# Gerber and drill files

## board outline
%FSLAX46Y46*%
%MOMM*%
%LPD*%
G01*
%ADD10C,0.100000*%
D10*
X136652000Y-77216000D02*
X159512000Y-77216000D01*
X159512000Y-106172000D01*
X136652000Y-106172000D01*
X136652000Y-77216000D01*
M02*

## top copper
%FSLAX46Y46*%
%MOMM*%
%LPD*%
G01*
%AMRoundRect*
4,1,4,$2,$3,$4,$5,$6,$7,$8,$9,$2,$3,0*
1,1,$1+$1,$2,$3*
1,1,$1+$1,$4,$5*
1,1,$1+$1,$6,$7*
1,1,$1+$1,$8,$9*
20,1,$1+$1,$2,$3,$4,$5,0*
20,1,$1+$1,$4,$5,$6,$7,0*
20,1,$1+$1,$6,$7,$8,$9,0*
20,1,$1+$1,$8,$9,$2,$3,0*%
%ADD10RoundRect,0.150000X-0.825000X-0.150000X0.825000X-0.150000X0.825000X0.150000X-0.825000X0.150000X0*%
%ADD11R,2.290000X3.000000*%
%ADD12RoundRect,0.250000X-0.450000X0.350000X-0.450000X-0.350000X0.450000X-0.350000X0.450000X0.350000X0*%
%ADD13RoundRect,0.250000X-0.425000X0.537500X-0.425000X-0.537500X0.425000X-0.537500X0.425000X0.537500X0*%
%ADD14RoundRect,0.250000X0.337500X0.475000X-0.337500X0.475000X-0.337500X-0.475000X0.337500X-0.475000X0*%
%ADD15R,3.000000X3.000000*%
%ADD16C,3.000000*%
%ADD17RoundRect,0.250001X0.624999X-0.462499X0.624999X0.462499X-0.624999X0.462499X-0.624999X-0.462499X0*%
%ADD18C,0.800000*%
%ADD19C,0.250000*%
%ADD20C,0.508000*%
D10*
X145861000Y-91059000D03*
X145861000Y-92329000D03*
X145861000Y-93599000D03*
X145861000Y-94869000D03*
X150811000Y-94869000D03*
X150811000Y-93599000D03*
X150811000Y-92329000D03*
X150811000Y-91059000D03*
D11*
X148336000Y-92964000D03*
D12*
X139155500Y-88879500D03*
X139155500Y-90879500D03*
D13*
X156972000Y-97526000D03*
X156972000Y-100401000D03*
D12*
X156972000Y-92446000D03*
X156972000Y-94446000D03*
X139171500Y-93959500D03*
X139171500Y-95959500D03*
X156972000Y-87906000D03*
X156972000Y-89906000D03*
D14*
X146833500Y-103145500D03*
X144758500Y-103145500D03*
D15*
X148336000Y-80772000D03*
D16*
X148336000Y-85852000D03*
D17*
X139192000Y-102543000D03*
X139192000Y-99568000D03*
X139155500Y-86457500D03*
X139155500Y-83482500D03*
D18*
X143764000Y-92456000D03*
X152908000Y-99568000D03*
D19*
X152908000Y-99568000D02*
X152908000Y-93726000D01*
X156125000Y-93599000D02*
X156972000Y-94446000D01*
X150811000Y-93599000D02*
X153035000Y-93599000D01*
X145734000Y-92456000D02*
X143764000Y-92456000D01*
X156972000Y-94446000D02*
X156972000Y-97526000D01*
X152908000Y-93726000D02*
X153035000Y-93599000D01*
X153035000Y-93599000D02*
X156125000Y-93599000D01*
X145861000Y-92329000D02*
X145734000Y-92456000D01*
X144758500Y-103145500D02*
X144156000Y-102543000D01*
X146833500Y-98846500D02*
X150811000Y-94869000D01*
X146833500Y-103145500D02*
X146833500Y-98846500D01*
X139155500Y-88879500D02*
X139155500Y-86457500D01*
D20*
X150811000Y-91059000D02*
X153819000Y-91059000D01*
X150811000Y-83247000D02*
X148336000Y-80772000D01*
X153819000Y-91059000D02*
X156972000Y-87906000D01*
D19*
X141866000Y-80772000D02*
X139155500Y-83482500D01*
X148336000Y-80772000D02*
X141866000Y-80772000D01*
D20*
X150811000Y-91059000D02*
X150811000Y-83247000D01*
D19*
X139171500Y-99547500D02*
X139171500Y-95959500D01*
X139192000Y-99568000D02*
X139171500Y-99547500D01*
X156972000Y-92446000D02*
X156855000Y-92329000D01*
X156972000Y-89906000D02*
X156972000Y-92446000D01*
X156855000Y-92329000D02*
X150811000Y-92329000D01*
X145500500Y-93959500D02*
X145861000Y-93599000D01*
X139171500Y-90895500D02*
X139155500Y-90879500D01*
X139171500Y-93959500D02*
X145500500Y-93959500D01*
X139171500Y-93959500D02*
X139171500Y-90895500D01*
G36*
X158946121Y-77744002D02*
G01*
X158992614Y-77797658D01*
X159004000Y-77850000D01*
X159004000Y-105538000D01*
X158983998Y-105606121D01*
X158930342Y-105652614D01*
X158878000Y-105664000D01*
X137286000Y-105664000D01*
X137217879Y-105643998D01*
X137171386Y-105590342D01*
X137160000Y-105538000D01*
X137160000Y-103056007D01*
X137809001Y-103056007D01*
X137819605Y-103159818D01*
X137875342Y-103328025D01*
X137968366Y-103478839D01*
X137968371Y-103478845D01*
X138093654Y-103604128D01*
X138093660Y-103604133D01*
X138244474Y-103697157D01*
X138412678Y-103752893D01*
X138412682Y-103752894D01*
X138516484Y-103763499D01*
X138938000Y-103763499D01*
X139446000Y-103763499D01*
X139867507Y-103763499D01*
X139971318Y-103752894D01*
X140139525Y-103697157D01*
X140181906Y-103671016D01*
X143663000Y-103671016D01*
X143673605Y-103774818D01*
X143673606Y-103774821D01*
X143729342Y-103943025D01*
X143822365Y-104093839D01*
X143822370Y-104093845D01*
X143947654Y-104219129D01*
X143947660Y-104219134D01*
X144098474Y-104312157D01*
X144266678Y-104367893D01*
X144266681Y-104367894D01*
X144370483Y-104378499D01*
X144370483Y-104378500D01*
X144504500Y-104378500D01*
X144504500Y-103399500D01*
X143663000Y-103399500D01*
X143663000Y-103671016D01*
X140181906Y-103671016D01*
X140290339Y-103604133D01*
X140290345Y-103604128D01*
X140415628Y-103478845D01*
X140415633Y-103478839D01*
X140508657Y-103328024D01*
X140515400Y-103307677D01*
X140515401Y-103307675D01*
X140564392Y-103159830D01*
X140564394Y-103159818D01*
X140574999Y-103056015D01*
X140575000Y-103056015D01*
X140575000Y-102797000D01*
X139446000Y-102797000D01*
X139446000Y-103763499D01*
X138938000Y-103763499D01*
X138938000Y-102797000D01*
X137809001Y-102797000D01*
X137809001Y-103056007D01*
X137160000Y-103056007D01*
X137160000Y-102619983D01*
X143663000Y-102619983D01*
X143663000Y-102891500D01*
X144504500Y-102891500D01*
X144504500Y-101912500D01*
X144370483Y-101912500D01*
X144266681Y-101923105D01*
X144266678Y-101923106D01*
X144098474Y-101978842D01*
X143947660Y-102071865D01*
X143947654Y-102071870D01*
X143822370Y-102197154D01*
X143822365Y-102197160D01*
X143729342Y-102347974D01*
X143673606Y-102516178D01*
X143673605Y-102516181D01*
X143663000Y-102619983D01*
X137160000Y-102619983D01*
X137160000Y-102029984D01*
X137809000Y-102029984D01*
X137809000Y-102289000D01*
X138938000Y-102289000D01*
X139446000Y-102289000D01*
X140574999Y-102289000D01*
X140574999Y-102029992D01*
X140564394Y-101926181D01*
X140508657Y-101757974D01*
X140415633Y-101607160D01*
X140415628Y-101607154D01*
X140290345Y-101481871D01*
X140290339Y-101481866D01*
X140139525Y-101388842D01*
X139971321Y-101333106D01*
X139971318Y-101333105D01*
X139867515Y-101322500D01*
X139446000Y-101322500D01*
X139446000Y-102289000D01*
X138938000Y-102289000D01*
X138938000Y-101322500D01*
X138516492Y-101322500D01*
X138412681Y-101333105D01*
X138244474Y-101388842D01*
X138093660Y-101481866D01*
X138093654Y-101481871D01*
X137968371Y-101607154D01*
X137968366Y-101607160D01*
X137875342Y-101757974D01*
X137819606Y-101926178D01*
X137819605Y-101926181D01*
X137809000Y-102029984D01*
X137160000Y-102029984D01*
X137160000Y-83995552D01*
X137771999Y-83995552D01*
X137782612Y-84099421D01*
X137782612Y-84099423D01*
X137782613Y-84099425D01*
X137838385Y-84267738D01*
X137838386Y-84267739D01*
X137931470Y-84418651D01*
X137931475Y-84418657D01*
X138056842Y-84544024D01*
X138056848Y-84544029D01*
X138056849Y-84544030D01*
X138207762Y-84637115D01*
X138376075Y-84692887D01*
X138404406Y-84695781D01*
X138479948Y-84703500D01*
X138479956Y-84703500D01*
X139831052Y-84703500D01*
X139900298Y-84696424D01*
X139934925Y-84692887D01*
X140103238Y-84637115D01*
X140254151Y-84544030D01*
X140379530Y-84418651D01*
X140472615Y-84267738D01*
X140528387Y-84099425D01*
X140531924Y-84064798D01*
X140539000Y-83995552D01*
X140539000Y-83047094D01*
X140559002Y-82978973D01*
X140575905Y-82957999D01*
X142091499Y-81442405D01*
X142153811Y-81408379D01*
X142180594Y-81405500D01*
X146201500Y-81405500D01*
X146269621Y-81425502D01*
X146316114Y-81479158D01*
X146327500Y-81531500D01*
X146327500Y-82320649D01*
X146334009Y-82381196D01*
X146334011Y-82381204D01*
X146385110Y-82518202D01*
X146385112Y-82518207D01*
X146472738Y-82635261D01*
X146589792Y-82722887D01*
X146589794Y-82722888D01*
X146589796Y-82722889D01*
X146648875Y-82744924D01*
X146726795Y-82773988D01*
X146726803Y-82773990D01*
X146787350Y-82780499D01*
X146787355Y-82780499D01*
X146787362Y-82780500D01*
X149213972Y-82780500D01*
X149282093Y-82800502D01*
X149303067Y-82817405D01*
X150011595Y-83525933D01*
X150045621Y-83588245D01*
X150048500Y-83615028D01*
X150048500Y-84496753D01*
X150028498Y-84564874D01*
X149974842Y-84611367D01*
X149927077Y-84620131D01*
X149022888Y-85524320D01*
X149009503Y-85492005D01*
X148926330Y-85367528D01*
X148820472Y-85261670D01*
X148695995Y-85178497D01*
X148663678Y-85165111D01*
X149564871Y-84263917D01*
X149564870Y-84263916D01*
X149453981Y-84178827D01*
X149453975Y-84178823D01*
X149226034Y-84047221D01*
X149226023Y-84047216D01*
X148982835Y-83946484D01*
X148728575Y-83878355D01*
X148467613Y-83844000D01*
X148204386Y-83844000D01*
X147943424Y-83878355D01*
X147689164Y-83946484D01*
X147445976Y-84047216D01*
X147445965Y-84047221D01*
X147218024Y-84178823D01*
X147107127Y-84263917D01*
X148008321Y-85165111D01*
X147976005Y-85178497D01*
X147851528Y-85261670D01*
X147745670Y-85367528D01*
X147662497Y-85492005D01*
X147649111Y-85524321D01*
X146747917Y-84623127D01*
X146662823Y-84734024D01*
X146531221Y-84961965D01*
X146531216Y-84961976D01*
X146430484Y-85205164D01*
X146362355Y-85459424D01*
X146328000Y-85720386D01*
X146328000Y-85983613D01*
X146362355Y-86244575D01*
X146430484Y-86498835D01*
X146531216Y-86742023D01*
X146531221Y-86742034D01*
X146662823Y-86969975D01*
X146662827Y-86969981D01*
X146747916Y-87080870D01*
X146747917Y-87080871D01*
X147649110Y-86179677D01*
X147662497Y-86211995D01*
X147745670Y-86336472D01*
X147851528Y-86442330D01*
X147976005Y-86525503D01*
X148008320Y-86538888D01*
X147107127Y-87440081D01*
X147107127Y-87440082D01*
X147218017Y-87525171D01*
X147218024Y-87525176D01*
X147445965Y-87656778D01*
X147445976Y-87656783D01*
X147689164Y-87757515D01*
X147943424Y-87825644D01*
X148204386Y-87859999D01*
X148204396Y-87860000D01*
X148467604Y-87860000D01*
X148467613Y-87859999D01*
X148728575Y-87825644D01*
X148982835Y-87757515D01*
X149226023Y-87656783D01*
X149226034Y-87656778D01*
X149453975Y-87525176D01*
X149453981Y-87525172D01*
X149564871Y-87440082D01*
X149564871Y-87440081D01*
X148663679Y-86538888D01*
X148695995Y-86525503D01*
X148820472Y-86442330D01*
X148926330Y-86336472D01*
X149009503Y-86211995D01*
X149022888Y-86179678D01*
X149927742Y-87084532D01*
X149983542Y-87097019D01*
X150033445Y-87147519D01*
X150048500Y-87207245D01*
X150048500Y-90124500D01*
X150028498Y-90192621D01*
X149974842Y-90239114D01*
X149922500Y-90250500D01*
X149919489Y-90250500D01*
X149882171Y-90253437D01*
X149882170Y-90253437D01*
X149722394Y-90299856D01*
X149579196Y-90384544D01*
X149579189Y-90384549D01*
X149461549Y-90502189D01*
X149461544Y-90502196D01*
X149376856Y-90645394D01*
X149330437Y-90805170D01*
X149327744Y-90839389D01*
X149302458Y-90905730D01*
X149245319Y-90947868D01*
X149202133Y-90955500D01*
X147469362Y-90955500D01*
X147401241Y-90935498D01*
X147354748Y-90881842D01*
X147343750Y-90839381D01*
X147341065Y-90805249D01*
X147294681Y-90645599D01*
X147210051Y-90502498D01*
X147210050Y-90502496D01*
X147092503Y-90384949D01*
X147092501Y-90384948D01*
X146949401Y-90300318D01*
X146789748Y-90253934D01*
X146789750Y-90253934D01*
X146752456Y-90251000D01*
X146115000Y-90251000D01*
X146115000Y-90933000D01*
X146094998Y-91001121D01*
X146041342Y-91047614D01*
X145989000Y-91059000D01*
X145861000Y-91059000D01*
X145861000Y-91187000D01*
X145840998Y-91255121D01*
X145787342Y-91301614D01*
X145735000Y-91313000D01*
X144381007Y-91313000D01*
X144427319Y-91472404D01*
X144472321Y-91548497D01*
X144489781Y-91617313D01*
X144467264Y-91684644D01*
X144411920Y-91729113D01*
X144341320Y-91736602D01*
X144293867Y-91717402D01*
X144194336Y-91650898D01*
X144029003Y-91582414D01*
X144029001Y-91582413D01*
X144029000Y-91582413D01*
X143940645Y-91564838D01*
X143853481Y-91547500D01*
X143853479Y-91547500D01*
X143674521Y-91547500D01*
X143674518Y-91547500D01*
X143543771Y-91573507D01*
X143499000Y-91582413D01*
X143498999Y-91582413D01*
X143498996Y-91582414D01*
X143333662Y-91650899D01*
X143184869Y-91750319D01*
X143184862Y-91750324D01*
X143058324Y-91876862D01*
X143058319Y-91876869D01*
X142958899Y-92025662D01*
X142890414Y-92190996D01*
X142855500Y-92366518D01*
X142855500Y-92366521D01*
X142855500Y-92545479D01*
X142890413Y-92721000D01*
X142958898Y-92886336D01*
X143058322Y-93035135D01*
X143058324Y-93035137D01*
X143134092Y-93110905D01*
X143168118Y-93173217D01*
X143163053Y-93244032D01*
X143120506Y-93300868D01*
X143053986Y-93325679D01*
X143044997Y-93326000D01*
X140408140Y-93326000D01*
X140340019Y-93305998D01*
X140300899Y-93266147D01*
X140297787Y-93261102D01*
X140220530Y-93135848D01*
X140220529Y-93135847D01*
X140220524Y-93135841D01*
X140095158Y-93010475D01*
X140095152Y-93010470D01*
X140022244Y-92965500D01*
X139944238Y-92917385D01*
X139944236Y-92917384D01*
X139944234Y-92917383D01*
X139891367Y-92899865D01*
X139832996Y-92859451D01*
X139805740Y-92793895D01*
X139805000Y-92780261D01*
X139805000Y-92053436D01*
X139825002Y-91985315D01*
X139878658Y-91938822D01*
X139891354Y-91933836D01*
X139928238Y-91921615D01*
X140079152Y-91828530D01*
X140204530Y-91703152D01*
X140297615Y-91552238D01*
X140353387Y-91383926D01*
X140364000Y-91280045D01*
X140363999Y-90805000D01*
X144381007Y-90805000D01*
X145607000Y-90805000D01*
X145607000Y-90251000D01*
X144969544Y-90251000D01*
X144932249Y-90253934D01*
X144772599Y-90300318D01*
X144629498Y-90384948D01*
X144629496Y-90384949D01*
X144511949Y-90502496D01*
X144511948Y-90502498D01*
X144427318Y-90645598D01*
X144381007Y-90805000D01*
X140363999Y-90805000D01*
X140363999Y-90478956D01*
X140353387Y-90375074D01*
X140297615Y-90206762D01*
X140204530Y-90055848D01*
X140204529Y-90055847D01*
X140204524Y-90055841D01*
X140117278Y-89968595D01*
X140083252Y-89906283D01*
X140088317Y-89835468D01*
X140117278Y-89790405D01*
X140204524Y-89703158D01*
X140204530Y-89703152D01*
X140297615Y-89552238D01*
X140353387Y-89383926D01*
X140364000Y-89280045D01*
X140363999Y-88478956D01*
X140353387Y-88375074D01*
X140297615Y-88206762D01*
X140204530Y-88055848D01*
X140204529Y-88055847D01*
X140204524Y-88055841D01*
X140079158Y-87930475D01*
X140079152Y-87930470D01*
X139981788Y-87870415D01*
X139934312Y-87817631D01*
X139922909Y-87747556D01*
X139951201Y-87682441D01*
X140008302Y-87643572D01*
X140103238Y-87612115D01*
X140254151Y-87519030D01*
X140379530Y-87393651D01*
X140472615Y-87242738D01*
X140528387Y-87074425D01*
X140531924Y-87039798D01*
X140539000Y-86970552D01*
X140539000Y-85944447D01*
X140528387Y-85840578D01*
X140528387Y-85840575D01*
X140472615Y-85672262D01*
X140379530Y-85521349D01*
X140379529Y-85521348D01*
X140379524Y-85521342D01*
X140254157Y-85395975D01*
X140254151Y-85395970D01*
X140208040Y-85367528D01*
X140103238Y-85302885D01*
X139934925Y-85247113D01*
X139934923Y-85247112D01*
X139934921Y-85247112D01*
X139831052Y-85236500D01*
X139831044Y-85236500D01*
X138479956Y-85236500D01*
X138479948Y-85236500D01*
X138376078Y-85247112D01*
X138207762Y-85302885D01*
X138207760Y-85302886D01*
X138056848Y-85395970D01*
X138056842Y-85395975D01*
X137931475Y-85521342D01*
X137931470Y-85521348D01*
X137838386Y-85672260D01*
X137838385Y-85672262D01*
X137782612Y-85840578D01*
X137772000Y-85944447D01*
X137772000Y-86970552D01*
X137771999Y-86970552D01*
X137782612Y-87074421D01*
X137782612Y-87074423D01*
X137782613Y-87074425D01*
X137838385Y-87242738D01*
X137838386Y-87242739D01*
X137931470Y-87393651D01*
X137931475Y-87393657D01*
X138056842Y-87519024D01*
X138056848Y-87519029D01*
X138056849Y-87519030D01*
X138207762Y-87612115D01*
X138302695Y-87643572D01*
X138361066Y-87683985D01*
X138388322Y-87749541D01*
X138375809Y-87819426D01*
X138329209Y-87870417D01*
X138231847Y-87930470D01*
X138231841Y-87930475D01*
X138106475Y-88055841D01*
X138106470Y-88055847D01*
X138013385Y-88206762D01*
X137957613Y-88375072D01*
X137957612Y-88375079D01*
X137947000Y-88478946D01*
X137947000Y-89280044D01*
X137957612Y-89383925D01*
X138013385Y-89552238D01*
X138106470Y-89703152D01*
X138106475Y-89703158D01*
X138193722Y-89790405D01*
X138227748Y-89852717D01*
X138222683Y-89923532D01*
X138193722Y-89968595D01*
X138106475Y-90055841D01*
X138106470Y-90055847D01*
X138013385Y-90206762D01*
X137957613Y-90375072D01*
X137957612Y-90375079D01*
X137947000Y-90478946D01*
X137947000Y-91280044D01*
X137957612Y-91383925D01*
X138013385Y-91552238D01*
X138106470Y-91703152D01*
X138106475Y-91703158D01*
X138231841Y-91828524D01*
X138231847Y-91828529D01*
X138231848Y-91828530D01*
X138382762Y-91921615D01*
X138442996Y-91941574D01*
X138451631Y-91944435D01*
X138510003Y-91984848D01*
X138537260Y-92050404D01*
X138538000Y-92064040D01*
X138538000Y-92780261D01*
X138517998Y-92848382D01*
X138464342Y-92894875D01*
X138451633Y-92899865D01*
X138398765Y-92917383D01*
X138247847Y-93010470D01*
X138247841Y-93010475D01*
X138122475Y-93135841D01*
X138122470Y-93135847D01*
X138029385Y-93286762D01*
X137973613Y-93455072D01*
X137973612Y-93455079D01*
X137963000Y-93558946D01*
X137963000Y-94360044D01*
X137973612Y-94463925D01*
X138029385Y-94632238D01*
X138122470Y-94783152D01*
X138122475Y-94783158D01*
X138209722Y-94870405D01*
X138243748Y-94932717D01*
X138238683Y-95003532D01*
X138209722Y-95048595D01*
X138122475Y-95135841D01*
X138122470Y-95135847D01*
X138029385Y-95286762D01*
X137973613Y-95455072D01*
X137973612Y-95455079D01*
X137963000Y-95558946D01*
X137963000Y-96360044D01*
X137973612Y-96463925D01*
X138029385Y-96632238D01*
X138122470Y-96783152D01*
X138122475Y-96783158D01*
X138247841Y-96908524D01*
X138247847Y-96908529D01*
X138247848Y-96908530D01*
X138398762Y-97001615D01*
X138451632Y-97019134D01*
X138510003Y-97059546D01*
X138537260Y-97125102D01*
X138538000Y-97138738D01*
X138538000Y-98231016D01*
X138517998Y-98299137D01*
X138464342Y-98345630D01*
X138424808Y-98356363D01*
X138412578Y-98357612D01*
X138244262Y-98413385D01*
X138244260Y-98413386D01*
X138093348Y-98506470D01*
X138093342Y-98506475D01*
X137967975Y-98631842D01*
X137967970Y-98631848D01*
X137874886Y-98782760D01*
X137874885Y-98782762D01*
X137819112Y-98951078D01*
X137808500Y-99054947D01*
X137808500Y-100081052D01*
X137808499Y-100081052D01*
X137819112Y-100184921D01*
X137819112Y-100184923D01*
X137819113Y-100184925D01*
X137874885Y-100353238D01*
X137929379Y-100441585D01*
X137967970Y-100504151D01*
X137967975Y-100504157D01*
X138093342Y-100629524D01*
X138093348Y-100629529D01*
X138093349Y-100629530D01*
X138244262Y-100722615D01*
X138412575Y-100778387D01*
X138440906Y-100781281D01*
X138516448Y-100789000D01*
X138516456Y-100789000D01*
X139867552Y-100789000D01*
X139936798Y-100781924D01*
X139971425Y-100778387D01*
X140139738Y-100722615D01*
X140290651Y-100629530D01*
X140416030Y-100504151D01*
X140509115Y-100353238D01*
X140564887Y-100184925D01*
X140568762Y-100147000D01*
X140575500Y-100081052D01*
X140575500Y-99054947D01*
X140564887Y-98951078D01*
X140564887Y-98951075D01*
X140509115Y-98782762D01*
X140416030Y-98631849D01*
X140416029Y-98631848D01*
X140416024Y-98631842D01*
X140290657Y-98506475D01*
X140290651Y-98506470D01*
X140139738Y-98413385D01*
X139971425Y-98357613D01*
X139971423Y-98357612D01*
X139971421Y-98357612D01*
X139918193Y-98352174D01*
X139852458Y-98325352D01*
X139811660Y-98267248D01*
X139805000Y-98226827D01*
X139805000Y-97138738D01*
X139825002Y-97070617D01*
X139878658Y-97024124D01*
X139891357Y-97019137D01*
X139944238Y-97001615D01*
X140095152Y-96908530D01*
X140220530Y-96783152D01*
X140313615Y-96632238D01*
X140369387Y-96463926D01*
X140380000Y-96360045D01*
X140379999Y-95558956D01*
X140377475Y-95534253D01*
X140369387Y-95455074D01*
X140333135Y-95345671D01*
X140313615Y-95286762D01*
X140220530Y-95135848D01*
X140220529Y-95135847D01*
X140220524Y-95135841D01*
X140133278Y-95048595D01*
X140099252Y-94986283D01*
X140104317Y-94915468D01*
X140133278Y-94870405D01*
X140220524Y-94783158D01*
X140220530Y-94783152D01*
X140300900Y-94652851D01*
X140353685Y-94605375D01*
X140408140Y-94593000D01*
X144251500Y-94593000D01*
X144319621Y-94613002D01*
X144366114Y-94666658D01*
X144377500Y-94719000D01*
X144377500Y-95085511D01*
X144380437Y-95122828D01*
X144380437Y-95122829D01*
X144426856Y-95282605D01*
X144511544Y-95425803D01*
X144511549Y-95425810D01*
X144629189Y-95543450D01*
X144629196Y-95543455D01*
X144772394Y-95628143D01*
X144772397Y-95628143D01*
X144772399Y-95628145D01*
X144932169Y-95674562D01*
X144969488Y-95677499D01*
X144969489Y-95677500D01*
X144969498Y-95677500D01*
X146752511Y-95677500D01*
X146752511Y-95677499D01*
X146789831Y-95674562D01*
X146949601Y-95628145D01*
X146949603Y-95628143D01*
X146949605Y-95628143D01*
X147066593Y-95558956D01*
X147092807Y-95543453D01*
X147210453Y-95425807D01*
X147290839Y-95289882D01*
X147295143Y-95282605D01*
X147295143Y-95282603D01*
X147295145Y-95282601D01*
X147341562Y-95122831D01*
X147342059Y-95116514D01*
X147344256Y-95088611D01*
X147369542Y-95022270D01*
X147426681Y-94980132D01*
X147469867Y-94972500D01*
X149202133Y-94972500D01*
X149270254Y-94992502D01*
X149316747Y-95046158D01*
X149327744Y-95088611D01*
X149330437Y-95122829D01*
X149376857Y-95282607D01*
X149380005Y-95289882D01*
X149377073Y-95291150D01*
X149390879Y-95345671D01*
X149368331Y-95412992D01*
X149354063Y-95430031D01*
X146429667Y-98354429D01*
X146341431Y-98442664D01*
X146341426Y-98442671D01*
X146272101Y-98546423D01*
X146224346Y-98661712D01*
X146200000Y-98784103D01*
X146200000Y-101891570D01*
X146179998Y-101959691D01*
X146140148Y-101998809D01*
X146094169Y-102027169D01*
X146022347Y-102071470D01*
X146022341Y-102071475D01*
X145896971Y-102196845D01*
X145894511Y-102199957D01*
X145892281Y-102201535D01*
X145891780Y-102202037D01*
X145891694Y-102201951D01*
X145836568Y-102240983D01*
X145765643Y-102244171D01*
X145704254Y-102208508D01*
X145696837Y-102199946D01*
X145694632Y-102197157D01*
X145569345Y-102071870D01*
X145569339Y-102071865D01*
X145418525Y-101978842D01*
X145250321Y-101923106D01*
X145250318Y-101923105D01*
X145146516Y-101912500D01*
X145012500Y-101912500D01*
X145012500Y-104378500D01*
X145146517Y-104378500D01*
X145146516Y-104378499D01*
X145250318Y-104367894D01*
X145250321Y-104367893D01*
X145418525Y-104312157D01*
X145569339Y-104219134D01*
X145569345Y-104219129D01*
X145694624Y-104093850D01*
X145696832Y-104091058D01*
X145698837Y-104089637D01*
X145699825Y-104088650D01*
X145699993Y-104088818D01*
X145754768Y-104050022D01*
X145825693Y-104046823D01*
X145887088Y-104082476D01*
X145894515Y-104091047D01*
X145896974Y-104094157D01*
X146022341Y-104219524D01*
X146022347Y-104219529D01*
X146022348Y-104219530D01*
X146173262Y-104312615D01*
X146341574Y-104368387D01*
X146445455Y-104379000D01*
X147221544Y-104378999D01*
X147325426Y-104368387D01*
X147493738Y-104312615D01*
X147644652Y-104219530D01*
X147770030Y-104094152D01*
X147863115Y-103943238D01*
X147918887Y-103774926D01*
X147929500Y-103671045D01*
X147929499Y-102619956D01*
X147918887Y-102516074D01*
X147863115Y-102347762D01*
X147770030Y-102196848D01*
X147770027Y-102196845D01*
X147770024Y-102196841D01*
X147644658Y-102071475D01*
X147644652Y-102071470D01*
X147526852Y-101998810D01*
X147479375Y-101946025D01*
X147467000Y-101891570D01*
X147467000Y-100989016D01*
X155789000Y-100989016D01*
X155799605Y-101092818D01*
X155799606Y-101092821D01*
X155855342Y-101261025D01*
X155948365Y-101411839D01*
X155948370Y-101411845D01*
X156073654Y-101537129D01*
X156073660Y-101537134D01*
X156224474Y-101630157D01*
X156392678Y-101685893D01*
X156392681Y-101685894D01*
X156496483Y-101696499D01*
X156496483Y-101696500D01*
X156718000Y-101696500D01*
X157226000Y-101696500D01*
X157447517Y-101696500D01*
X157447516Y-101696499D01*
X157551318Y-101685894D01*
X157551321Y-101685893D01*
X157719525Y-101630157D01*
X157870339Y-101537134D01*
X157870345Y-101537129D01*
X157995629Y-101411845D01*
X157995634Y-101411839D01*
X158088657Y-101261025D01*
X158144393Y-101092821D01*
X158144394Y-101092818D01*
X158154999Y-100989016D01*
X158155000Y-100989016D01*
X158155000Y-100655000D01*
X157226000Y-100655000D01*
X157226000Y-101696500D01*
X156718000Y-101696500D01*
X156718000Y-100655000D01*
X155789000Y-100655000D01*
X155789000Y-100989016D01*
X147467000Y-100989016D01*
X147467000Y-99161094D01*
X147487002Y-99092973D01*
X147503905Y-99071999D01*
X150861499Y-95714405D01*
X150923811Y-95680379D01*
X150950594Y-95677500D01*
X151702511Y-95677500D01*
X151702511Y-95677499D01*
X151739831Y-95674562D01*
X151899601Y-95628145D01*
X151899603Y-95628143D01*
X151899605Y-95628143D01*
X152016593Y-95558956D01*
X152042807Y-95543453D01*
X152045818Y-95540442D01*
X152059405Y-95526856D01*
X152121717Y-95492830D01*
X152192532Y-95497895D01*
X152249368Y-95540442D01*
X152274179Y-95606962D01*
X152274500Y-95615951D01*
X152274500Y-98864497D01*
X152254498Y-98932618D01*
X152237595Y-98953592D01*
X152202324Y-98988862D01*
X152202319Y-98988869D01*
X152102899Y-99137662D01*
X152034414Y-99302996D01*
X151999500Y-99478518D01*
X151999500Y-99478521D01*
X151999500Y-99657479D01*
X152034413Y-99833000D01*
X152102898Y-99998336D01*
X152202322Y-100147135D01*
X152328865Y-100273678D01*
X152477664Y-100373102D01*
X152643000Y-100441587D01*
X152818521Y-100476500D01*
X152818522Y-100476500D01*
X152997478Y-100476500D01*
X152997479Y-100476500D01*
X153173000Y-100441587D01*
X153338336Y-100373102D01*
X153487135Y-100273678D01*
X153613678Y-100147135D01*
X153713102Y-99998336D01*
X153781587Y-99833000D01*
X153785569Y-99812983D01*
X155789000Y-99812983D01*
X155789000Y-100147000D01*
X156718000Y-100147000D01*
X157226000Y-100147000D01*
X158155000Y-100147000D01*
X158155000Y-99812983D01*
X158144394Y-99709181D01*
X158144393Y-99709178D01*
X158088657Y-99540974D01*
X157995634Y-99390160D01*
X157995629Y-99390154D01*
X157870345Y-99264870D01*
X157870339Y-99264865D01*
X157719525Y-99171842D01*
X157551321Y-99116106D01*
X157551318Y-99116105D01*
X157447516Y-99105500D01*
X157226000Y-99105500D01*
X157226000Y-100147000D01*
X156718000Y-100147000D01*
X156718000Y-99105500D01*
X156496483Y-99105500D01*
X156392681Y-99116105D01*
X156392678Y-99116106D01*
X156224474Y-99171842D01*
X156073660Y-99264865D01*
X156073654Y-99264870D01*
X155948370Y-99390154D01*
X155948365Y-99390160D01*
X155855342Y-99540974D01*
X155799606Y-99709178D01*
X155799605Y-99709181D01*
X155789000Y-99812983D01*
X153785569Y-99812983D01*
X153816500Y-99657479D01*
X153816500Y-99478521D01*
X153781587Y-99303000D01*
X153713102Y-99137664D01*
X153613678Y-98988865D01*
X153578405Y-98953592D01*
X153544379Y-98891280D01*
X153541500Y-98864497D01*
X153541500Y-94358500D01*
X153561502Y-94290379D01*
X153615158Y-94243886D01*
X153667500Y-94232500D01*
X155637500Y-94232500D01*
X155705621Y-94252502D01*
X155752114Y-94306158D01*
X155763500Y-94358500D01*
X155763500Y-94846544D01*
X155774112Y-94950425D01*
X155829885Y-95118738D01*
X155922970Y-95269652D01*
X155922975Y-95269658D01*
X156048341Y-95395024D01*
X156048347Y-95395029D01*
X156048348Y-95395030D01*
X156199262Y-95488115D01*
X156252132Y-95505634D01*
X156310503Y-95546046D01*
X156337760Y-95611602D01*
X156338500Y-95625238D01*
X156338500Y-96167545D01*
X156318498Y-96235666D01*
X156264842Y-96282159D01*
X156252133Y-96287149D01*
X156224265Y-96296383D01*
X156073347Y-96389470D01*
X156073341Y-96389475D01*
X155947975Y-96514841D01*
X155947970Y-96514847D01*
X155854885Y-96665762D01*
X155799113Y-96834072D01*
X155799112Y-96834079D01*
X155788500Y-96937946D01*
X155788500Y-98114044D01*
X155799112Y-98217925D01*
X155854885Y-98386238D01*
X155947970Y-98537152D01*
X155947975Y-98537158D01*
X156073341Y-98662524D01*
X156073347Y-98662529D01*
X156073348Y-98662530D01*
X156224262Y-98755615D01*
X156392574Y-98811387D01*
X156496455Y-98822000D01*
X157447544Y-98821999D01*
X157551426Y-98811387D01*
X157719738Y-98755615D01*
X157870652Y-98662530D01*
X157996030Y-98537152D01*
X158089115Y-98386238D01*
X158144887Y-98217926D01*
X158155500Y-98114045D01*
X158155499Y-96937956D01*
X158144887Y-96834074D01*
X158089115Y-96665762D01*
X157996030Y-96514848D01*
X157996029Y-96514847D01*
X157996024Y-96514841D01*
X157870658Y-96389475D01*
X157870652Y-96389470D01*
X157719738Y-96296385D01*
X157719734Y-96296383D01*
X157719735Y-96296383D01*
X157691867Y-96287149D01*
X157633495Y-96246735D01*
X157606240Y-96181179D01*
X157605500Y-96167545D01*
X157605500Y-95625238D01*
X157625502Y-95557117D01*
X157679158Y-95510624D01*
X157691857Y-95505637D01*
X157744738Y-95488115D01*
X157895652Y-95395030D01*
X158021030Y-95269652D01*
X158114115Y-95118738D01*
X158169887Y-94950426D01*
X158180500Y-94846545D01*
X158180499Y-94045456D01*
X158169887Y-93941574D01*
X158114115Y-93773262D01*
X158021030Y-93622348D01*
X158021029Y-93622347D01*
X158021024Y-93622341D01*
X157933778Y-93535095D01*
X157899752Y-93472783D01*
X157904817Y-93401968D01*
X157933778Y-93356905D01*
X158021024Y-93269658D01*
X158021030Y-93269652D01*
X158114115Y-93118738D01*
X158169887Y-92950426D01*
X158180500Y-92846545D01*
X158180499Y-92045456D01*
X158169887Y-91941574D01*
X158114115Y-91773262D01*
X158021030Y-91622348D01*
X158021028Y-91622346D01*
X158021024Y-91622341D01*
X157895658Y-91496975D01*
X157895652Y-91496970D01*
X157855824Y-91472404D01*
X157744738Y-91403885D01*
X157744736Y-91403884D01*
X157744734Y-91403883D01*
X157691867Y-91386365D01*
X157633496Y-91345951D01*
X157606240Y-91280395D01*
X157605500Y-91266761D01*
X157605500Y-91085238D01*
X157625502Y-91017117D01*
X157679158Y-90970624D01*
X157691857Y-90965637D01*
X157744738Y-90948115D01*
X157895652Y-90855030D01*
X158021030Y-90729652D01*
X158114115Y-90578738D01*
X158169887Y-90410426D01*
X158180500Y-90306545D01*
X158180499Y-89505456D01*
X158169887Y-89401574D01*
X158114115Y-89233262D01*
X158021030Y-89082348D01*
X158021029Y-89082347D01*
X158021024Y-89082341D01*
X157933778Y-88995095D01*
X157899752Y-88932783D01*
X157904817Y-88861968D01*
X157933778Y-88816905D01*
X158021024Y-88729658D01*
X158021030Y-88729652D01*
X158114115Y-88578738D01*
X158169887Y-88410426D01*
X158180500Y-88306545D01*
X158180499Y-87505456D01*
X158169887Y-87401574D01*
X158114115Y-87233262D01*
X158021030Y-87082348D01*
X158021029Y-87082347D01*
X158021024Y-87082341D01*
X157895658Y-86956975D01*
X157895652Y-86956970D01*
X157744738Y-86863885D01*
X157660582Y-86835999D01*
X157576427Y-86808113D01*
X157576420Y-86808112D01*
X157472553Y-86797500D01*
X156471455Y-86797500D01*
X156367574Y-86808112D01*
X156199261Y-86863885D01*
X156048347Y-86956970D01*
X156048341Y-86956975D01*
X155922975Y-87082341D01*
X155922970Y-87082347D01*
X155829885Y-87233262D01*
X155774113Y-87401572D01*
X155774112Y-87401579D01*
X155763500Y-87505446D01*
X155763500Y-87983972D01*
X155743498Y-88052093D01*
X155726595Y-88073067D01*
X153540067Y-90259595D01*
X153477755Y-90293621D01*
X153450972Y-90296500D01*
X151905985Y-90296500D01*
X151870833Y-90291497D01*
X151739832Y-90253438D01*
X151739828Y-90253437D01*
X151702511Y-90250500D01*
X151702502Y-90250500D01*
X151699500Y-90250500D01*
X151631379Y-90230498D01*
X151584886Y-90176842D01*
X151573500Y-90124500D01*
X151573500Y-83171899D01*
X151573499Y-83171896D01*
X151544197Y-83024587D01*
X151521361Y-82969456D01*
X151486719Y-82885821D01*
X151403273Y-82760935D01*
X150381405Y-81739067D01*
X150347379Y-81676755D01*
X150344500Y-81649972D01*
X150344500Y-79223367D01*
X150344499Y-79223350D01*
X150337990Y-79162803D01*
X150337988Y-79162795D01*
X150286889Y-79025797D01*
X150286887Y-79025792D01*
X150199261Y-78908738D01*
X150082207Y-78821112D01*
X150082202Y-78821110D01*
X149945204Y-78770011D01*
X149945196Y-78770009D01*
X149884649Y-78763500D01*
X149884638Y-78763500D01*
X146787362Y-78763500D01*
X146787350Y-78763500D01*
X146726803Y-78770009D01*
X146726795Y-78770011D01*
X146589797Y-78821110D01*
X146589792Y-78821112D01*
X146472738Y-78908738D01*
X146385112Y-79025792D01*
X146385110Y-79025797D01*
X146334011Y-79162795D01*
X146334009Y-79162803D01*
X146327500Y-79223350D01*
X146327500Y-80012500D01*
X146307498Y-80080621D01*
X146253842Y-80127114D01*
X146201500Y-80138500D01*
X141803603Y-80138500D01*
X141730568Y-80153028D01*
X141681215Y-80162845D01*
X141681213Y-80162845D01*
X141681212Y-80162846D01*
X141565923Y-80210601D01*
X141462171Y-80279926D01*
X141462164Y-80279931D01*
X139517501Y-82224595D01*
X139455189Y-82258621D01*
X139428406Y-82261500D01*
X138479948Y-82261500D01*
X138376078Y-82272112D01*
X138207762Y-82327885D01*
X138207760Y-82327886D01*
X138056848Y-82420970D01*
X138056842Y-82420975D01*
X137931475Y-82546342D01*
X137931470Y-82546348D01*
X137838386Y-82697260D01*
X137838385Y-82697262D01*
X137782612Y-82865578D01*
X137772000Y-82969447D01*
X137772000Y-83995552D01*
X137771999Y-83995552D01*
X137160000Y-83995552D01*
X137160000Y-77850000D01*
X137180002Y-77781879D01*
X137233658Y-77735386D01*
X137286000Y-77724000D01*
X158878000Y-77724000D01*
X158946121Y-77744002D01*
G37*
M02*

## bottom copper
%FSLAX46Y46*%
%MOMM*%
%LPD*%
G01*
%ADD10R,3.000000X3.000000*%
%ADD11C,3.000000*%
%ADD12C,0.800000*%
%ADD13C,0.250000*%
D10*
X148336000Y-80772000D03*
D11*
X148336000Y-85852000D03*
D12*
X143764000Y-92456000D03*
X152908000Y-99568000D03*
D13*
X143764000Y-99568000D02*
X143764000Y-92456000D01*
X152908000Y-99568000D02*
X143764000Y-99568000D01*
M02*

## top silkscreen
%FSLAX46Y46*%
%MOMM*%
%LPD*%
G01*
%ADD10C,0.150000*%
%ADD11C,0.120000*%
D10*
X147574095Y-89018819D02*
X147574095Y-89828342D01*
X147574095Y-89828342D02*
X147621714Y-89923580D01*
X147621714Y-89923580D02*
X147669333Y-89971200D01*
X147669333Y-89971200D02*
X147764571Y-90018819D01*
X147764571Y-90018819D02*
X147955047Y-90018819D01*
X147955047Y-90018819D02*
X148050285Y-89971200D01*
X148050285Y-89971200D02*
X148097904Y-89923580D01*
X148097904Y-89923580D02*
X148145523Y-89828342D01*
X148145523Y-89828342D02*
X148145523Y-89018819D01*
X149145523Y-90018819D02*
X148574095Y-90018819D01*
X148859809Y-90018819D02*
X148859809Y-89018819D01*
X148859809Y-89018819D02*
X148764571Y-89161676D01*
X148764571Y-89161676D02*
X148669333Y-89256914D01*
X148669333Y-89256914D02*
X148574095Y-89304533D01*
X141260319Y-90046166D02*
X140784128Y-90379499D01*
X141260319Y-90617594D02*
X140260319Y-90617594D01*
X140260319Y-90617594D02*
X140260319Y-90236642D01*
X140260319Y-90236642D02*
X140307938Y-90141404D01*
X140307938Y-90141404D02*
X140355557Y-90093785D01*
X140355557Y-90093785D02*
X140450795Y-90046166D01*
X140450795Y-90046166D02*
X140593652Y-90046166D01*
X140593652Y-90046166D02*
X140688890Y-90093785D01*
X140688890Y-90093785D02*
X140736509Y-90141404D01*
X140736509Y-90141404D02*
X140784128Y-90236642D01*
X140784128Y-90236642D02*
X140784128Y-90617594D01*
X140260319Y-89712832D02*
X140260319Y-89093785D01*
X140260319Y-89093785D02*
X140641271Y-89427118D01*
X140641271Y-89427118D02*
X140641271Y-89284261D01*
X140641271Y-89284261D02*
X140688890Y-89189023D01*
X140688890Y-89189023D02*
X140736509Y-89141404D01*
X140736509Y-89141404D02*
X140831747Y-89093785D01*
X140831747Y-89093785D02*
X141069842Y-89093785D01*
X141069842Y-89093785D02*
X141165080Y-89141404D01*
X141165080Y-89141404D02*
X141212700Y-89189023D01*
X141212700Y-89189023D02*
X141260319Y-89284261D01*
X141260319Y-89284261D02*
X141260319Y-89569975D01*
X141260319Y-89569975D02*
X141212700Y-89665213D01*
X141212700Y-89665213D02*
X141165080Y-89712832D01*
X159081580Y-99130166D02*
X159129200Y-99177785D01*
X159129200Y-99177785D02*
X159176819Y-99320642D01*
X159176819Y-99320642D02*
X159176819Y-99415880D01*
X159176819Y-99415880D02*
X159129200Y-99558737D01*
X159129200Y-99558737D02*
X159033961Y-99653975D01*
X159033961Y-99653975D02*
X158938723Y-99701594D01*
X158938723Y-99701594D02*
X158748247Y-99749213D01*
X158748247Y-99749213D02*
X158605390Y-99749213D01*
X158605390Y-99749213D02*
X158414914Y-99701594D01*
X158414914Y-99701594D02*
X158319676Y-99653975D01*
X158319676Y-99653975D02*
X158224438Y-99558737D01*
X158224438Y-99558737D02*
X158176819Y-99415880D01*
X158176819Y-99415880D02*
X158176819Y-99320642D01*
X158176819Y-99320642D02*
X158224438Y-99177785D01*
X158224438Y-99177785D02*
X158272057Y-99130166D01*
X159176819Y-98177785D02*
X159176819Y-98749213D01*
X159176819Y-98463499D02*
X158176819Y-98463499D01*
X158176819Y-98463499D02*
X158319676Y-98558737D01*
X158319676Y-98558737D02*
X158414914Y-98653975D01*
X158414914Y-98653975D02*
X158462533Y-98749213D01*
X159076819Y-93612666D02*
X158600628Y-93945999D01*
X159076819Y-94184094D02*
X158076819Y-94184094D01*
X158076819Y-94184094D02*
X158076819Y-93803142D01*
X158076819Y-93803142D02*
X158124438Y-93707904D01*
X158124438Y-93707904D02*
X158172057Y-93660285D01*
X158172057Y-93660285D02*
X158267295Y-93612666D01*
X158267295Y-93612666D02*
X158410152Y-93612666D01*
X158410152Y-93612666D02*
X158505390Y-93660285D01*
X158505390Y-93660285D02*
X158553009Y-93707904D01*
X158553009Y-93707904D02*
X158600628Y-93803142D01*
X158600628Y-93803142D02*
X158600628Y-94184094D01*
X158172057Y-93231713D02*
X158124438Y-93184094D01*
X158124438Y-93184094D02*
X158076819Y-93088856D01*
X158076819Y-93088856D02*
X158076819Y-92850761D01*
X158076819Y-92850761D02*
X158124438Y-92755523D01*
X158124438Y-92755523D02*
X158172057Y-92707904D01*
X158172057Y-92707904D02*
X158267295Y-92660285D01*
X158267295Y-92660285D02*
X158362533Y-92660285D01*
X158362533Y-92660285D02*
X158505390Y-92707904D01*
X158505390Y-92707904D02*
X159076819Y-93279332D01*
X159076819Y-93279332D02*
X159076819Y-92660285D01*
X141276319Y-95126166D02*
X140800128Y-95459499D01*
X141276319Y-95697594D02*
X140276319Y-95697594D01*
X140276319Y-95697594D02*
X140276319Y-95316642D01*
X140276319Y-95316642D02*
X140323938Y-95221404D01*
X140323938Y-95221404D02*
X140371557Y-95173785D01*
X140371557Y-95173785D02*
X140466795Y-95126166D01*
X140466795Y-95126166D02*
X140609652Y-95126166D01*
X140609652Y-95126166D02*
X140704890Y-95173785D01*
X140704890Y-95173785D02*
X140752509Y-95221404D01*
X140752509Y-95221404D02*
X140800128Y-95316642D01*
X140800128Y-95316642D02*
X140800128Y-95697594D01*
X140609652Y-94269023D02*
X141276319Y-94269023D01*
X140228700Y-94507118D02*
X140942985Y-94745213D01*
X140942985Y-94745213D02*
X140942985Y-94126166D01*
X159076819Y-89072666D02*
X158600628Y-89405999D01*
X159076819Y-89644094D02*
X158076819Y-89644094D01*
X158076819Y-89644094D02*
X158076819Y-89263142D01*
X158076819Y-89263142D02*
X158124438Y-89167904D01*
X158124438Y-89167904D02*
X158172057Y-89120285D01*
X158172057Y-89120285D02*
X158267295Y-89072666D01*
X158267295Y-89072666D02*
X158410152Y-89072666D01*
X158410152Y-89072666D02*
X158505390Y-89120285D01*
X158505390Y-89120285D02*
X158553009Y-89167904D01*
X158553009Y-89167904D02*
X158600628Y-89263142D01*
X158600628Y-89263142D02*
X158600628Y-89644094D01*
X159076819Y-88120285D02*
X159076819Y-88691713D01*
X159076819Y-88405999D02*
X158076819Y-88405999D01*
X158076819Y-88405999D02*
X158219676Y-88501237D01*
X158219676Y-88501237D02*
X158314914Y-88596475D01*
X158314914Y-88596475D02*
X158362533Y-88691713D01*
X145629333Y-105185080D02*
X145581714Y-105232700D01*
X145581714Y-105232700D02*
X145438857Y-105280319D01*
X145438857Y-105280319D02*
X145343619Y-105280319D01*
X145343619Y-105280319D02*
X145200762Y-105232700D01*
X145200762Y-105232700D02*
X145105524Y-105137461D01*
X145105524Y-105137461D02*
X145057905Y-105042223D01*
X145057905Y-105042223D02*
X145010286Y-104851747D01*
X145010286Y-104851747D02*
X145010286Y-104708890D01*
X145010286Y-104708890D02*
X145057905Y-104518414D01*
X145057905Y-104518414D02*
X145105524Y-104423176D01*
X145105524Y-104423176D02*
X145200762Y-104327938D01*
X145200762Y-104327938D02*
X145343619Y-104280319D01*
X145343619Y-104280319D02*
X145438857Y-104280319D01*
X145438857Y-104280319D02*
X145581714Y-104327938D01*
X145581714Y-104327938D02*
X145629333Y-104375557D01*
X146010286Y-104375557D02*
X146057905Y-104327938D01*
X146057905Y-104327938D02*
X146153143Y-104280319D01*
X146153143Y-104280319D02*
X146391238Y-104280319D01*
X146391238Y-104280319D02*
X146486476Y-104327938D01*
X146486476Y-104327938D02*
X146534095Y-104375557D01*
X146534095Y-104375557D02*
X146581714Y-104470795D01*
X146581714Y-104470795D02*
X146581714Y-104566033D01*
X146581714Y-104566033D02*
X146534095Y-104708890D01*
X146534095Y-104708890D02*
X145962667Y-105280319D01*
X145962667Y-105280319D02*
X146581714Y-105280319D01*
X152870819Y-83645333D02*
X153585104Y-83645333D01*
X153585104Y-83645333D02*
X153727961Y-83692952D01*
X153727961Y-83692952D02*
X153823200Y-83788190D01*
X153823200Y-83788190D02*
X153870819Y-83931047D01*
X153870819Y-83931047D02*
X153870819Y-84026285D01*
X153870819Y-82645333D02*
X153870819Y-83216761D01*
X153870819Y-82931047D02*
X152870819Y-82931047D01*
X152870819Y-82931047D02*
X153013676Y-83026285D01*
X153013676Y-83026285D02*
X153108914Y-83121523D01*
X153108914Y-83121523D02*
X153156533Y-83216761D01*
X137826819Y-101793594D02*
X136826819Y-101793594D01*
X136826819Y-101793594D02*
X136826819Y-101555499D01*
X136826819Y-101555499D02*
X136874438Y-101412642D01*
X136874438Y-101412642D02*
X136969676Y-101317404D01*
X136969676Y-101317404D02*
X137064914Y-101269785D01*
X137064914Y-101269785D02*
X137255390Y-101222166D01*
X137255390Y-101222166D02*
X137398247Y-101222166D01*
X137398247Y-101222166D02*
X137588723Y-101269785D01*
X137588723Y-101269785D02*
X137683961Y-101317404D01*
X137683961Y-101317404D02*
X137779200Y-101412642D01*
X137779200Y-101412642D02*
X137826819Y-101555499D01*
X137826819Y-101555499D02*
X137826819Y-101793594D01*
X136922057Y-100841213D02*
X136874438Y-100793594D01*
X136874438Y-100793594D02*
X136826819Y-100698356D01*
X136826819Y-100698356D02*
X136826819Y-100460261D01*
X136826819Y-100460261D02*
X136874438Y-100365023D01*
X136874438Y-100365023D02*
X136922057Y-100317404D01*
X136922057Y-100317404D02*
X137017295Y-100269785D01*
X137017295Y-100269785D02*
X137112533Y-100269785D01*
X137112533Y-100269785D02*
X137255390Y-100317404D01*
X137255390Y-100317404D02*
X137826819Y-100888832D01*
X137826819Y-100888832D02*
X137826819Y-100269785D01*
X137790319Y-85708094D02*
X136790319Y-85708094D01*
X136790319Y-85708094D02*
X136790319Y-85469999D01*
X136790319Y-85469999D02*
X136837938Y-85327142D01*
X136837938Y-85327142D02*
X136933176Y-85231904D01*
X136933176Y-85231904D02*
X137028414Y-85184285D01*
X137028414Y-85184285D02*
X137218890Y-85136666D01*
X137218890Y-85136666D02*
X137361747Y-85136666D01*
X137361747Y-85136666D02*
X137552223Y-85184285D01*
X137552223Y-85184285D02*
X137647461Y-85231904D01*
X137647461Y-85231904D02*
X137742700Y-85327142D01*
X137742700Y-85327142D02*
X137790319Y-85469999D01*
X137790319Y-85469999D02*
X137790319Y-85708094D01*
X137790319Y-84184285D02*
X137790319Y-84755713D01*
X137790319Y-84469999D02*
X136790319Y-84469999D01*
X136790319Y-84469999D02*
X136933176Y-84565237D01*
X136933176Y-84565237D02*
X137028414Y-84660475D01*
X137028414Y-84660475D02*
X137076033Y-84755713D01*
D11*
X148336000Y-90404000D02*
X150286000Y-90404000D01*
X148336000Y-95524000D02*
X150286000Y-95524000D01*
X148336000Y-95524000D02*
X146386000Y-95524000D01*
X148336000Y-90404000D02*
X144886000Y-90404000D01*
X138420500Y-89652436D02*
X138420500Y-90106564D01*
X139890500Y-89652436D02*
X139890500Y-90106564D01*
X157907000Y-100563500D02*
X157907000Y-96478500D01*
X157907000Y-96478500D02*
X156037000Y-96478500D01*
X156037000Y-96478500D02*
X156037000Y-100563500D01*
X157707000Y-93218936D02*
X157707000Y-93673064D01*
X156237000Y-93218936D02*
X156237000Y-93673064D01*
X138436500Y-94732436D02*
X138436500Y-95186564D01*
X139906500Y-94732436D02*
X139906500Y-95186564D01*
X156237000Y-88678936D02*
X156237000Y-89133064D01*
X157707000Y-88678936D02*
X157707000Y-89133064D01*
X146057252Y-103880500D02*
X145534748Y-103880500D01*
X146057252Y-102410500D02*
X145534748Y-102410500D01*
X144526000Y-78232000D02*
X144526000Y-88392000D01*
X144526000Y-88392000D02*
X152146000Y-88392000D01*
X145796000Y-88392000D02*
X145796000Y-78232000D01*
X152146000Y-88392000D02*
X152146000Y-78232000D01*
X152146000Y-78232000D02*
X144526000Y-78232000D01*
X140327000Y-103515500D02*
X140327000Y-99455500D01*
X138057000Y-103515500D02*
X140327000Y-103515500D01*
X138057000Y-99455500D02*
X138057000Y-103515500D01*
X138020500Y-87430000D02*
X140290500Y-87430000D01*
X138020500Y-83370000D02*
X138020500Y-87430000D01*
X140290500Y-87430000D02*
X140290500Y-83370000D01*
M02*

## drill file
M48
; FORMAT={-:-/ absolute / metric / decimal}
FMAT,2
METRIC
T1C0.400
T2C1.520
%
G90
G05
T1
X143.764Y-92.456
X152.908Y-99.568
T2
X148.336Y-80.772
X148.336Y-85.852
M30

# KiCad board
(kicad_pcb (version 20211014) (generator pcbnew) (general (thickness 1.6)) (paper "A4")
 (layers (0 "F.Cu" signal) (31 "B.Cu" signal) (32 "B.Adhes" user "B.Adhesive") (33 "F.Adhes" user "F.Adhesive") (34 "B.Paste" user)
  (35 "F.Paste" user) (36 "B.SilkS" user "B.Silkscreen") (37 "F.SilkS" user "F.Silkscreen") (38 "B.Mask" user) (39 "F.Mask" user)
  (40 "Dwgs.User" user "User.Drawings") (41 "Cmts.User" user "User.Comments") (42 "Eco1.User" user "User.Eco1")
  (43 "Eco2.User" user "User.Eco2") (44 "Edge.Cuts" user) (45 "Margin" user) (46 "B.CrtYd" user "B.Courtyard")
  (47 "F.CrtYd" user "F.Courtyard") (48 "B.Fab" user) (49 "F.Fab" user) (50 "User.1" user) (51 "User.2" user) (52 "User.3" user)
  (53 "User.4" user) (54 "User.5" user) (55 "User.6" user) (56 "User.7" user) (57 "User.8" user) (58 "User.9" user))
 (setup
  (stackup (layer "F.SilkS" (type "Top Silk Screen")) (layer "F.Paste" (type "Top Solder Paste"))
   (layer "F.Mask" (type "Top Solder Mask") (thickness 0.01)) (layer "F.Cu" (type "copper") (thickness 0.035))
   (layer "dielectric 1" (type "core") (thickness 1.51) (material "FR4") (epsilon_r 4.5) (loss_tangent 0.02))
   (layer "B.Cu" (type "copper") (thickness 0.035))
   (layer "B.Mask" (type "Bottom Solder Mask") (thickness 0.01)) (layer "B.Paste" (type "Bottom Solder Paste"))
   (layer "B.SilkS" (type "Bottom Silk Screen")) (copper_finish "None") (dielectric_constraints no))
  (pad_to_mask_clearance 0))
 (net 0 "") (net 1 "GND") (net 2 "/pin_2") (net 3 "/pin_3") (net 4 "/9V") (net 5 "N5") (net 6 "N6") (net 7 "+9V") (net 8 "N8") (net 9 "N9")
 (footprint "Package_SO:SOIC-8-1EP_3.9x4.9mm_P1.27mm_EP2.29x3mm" (layer "F.Cu") (at 148.336 92.964)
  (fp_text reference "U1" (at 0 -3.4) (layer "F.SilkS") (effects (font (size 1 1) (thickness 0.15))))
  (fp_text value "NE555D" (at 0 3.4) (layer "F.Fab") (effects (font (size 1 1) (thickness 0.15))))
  (fp_line (start 0 -2.56) (end 1.95 -2.56) (layer "F.SilkS") (width 0.12))
  (fp_line (start 0 2.56) (end 1.95 2.56) (layer "F.SilkS") (width 0.12))
  (fp_line (start 0 2.56) (end -1.95 2.56) (layer "F.SilkS") (width 0.12))
  (fp_line (start 0 -2.56) (end -3.45 -2.56) (layer "F.SilkS") (width 0.12))
  (pad "" smd roundrect (at 0.57 0.75) (size 0.92 1.21) (layers "F.Paste") (roundrect_rratio 0.25))
  (pad "" smd roundrect (at 0.57 -0.75) (size 0.92 1.21) (layers "F.Paste") (roundrect_rratio 0.25))
  (pad "" smd roundrect (at -0.57 0.75) (size 0.92 1.21) (layers "F.Paste") (roundrect_rratio 0.25))
  (pad "" smd roundrect (at -0.57 -0.75) (size 0.92 1.21) (layers "F.Paste") (roundrect_rratio 0.25))
  (pad "1" smd roundrect (at -2.475 -1.905) (size 1.95 0.6) (layers "F.Cu" "F.Paste" "F.Mask") (roundrect_rratio 0.25) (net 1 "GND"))
  (pad "2" smd roundrect (at -2.475 -0.635) (size 1.95 0.6) (layers "F.Cu" "F.Paste" "F.Mask") (roundrect_rratio 0.25) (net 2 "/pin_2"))
  (pad "3" smd roundrect (at -2.475 0.635) (size 1.95 0.6) (layers "F.Cu" "F.Paste" "F.Mask") (roundrect_rratio 0.25) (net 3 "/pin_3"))
  (pad "4" smd roundrect (at -2.475 1.905) (size 1.95 0.6) (layers "F.Cu" "F.Paste" "F.Mask") (roundrect_rratio 0.25) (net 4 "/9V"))
  (pad "5" smd roundrect (at 2.475 1.905) (size 1.95 0.6) (layers "F.Cu" "F.Paste" "F.Mask") (roundrect_rratio 0.25) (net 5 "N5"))
  (pad "6" smd roundrect (at 2.475 0.635) (size 1.95 0.6) (layers "F.Cu" "F.Paste" "F.Mask") (roundrect_rratio 0.25) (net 2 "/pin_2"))
  (pad "7" smd roundrect (at 2.475 -0.635) (size 1.95 0.6) (layers "F.Cu" "F.Paste" "F.Mask") (roundrect_rratio 0.25) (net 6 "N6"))
  (pad "8" smd roundrect (at 2.475 -1.905) (size 1.95 0.6) (layers "F.Cu" "F.Paste" "F.Mask") (roundrect_rratio 0.25) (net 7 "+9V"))
  (pad "9" smd rect (at 0 0) (size 2.29 3) (layers "F.Cu" "F.Mask")))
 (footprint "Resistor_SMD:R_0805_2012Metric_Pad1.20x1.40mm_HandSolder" (layer "F.Cu") (at 139.1555 89.8795 -90)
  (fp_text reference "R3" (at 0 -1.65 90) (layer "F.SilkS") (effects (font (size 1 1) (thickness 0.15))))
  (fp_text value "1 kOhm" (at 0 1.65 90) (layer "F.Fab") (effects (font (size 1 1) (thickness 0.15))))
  (fp_line (start -0.227064 0.735) (end 0.227064 0.735) (layer "F.SilkS") (width 0.12))
  (fp_line (start -0.227064 -0.735) (end 0.227064 -0.735) (layer "F.SilkS") (width 0.12))
  (pad "1" smd roundrect (at -1 0 270) (size 1.2 1.4) (layers "F.Cu" "F.Paste" "F.Mask") (roundrect_rratio 0.2083333333) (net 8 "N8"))
  (pad "2" smd roundrect (at 1 0 270) (size 1.2 1.4) (layers "F.Cu" "F.Paste" "F.Mask") (roundrect_rratio 0.2083333333) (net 3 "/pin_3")))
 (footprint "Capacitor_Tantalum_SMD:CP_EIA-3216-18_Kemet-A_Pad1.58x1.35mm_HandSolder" (layer "F.Cu") (at 156.972 98.9635 -90)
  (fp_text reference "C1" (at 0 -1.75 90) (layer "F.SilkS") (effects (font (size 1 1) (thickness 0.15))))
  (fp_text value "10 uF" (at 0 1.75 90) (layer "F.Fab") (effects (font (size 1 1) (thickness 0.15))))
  (fp_line (start 1.6 -0.935) (end -2.485 -0.935) (layer "F.SilkS") (width 0.12))
  (fp_line (start -2.485 -0.935) (end -2.485 0.935) (layer "F.SilkS") (width 0.12))
  (fp_line (start -2.485 0.935) (end 1.6 0.935) (layer "F.SilkS") (width 0.12))
  (pad "1" smd roundrect (at -1.4375 0 270) (size 1.575 1.35) (layers "F.Cu" "F.Paste" "F.Mask") (roundrect_rratio 0.1851851852)
   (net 2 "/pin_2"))
  (pad "2" smd roundrect (at 1.4375 0 270) (size 1.575 1.35) (layers "F.Cu" "F.Paste" "F.Mask") (roundrect_rratio 0.1851851852)
   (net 1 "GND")))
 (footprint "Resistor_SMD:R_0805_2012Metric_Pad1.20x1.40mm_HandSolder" (layer "F.Cu") (at 156.972 93.446 -90)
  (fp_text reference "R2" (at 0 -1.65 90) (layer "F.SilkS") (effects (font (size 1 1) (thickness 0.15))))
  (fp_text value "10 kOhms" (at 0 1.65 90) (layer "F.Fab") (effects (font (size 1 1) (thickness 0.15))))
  (fp_line (start -0.227064 -0.735) (end 0.227064 -0.735) (layer "F.SilkS") (width 0.12))
  (fp_line (start -0.227064 0.735) (end 0.227064 0.735) (layer "F.SilkS") (width 0.12))
  (pad "1" smd roundrect (at -1 0 270) (size 1.2 1.4) (layers "F.Cu" "F.Paste" "F.Mask") (roundrect_rratio 0.2083333333) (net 6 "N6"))
  (pad "2" smd roundrect (at 1 0 270) (size 1.2 1.4) (layers "F.Cu" "F.Paste" "F.Mask") (roundrect_rratio 0.2083333333) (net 2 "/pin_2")))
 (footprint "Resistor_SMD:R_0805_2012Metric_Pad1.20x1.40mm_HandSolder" (layer "F.Cu") (at 139.1715 94.9595 -90)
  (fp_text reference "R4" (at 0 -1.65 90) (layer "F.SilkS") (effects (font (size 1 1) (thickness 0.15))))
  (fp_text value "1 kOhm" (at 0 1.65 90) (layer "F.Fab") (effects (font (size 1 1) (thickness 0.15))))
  (fp_line (start -0.227064 0.735) (end 0.227064 0.735) (layer "F.SilkS") (width 0.12))
  (fp_line (start -0.227064 -0.735) (end 0.227064 -0.735) (layer "F.SilkS") (width 0.12))
  (pad "1" smd roundrect (at -1 0 270) (size 1.2 1.4) (layers "F.Cu" "F.Paste" "F.Mask") (roundrect_rratio 0.2083333333) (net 3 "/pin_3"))
  (pad "2" smd roundrect (at 1 0 270) (size 1.2 1.4) (layers "F.Cu" "F.Paste" "F.Mask") (roundrect_rratio 0.2083333333) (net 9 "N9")))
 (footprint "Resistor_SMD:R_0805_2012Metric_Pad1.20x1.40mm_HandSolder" (layer "F.Cu") (at 156.972 88.906 -90)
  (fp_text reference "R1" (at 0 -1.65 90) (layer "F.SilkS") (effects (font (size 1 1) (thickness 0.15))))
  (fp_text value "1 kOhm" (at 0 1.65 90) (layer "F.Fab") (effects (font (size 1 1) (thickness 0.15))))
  (fp_line (start -0.227064 0.735) (end 0.227064 0.735) (layer "F.SilkS") (width 0.12))
  (fp_line (start -0.227064 -0.735) (end 0.227064 -0.735) (layer "F.SilkS") (width 0.12))
  (pad "1" smd roundrect (at -1 0 270) (size 1.2 1.4) (layers "F.Cu" "F.Paste" "F.Mask") (roundrect_rratio 0.2083333333) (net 7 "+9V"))
  (pad "2" smd roundrect (at 1 0 270) (size 1.2 1.4) (layers "F.Cu" "F.Paste" "F.Mask") (roundrect_rratio 0.2083333333) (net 6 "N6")))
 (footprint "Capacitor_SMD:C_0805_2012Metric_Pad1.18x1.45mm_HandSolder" (layer "F.Cu") (at 145.796 103.1455 180)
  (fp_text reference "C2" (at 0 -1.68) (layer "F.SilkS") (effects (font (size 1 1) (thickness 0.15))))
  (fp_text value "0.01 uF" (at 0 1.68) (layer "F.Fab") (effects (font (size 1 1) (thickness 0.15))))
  (fp_line (start -0.261252 -0.735) (end 0.261252 -0.735) (layer "F.SilkS") (width 0.12))
  (fp_line (start -0.261252 0.735) (end 0.261252 0.735) (layer "F.SilkS") (width 0.12))
  (pad "1" smd roundrect (at -1.0375 0 180) (size 1.175 1.45) (layers "F.Cu" "F.Paste" "F.Mask") (roundrect_rratio 0.2127659574)
   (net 5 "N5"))
  (pad "2" smd roundrect (at 1.0375 0 180) (size 1.175 1.45) (layers "F.Cu" "F.Paste" "F.Mask") (roundrect_rratio 0.2127659574)
   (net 1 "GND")))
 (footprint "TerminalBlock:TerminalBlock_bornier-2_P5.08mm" (layer "F.Cu") (at 148.336 80.772 -90)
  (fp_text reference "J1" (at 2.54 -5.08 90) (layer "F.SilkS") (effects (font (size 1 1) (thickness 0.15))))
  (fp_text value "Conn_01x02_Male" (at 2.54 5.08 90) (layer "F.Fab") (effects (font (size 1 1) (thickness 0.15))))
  (fp_line (start -2.54 3.81) (end 7.62 3.81) (layer "F.SilkS") (width 0.12))
  (fp_line (start 7.62 3.81) (end 7.62 -3.81) (layer "F.SilkS") (width 0.12))
  (fp_line (start 7.62 2.54) (end -2.54 2.54) (layer "F.SilkS") (width 0.12))
  (fp_line (start 7.62 -3.81) (end -2.54 -3.81) (layer "F.SilkS") (width 0.12))
  (fp_line (start -2.54 -3.81) (end -2.54 3.81) (layer "F.SilkS") (width 0.12))
  (pad "1" thru_hole rect (at 0 0 270) (size 3 3) (drill 1.52) (layers *.Cu *.Mask) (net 7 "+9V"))
  (pad "2" thru_hole circle (at 5.08 0 270) (size 3 3) (drill 1.52) (layers *.Cu *.Mask) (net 1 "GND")))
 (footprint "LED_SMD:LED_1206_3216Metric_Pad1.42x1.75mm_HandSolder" (layer "F.Cu") (at 139.192 101.0555 90)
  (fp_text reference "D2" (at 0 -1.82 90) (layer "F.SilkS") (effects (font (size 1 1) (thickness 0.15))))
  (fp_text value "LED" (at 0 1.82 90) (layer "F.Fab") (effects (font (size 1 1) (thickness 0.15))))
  (fp_line (start -2.46 1.135) (end 1.6 1.135) (layer "F.SilkS") (width 0.12))
  (fp_line (start -2.46 -1.135) (end -2.46 1.135) (layer "F.SilkS") (width 0.12))
  (fp_line (start 1.6 -1.135) (end -2.46 -1.135) (layer "F.SilkS") (width 0.12))
  (pad "1" smd roundrect (at -1.4875 0 90) (size 1.425 1.75) (layers "F.Cu" "F.Paste" "F.Mask") (roundrect_rratio 0.1754392982)
   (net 1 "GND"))
  (pad "2" smd roundrect (at 1.4875 0 90) (size 1.425 1.75) (layers "F.Cu" "F.Paste" "F.Mask") (roundrect_rratio 0.1754392982) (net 9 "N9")))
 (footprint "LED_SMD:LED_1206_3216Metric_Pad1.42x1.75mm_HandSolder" (layer "F.Cu") (at 139.1555 84.97 90)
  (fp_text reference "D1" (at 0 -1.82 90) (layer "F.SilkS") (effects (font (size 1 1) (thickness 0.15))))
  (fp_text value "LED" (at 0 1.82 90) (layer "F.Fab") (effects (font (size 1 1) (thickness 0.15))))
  (fp_line (start -2.46 -1.135) (end -2.46 1.135) (layer "F.SilkS") (width 0.12))
  (fp_line (start 1.6 -1.135) (end -2.46 -1.135) (layer "F.SilkS") (width 0.12))
  (fp_line (start -2.46 1.135) (end 1.6 1.135) (layer "F.SilkS") (width 0.12))
  (pad "1" smd roundrect (at -1.4875 0 90) (size 1.425 1.75) (layers "F.Cu" "F.Paste" "F.Mask") (roundrect_rratio 0.1754392982) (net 8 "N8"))
  (pad "2" smd roundrect (at 1.4875 0 90) (size 1.425 1.75) (layers "F.Cu" "F.Paste" "F.Mask") (roundrect_rratio 0.1754392982) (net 7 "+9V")))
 (gr_rect (start 136.652 106.172) (end 159.512 77.216) (layer "Edge.Cuts") (width 0.1) (fill none))
 (segment (start 152.908 99.568) (end 152.908 93.726) (width 0.25) (layer "F.Cu") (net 2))
 (segment (start 156.125 93.599) (end 156.972 94.446) (width 0.25) (layer "F.Cu") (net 2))
 (segment (start 150.811 93.599) (end 153.035 93.599) (width 0.25) (layer "F.Cu") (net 2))
 (segment (start 145.734 92.456) (end 143.764 92.456) (width 0.25) (layer "F.Cu") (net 2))
 (segment (start 156.972 94.446) (end 156.972 97.526) (width 0.25) (layer "F.Cu") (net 2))
 (segment (start 152.908 93.726) (end 153.035 93.599) (width 0.25) (layer "F.Cu") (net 2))
 (segment (start 153.035 93.599) (end 156.125 93.599) (width 0.25) (layer "F.Cu") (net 2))
 (segment (start 145.861 92.329) (end 145.734 92.456) (width 0.25) (layer "F.Cu") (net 2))
 (via (at 143.764 92.456) (size 0.8) (drill 0.4) (layers "F.Cu" "B.Cu") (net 2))
 (via (at 152.908 99.568) (size 0.8) (drill 0.4) (layers "F.Cu" "B.Cu") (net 2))
 (segment (start 143.764 99.568) (end 143.764 92.456) (width 0.25) (layer "B.Cu") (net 2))
 (segment (start 152.908 99.568) (end 143.764 99.568) (width 0.25) (layer "B.Cu") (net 2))
 (segment (start 144.7585 103.1455) (end 144.156 102.543) (width 0.25) (layer "F.Cu") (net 1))
 (segment (start 146.8335 98.8465) (end 150.811 94.869) (width 0.25) (layer "F.Cu") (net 5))
 (segment (start 146.8335 103.1455) (end 146.8335 98.8465) (width 0.25) (layer "F.Cu") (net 5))
 (segment (start 139.1555 88.8795) (end 139.1555 86.4575) (width 0.25) (layer "F.Cu") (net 8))
 (segment (start 150.811 91.059) (end 153.819 91.059) (width 0.508) (layer "F.Cu") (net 7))
 (segment (start 150.811 83.247) (end 148.336 80.772) (width 0.508) (layer "F.Cu") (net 7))
 (segment (start 153.819 91.059) (end 156.972 87.906) (width 0.508) (layer "F.Cu") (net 7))
 (segment (start 141.866 80.772) (end 139.1555 83.4825) (width 0.25) (layer "F.Cu") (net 7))
 (segment (start 148.336 80.772) (end 141.866 80.772) (width 0.25) (layer "F.Cu") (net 7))
 (segment (start 150.811 91.059) (end 150.811 83.247) (width 0.508) (layer "F.Cu") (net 7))
 (segment (start 139.1715 99.5475) (end 139.1715 95.9595) (width 0.25) (layer "F.Cu") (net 9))
 (segment (start 139.192 99.568) (end 139.1715 99.5475) (width 0.25) (layer "F.Cu") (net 9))
 (segment (start 156.972 92.446) (end 156.855 92.329) (width 0.25) (layer "F.Cu") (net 6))
 (segment (start 156.972 89.906) (end 156.972 92.446) (width 0.25) (layer "F.Cu") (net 6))
 (segment (start 156.855 92.329) (end 150.811 92.329) (width 0.25) (layer "F.Cu") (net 6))
 (segment (start 145.5005 93.9595) (end 145.861 93.599) (width 0.25) (layer "F.Cu") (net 3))
 (segment (start 139.1715 90.8955) (end 139.1555 90.8795) (width 0.25) (layer "F.Cu") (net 3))
 (segment (start 139.1715 93.9595) (end 145.5005 93.9595) (width 0.25) (layer "F.Cu") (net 3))
 (segment (start 139.1715 93.9595) (end 139.1715 90.8955) (width 0.25) (layer "F.Cu") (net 3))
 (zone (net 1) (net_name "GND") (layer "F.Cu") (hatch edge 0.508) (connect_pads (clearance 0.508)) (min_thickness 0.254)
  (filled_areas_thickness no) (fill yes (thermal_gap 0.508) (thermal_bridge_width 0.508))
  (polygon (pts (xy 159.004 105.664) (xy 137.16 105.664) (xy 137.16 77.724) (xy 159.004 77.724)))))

